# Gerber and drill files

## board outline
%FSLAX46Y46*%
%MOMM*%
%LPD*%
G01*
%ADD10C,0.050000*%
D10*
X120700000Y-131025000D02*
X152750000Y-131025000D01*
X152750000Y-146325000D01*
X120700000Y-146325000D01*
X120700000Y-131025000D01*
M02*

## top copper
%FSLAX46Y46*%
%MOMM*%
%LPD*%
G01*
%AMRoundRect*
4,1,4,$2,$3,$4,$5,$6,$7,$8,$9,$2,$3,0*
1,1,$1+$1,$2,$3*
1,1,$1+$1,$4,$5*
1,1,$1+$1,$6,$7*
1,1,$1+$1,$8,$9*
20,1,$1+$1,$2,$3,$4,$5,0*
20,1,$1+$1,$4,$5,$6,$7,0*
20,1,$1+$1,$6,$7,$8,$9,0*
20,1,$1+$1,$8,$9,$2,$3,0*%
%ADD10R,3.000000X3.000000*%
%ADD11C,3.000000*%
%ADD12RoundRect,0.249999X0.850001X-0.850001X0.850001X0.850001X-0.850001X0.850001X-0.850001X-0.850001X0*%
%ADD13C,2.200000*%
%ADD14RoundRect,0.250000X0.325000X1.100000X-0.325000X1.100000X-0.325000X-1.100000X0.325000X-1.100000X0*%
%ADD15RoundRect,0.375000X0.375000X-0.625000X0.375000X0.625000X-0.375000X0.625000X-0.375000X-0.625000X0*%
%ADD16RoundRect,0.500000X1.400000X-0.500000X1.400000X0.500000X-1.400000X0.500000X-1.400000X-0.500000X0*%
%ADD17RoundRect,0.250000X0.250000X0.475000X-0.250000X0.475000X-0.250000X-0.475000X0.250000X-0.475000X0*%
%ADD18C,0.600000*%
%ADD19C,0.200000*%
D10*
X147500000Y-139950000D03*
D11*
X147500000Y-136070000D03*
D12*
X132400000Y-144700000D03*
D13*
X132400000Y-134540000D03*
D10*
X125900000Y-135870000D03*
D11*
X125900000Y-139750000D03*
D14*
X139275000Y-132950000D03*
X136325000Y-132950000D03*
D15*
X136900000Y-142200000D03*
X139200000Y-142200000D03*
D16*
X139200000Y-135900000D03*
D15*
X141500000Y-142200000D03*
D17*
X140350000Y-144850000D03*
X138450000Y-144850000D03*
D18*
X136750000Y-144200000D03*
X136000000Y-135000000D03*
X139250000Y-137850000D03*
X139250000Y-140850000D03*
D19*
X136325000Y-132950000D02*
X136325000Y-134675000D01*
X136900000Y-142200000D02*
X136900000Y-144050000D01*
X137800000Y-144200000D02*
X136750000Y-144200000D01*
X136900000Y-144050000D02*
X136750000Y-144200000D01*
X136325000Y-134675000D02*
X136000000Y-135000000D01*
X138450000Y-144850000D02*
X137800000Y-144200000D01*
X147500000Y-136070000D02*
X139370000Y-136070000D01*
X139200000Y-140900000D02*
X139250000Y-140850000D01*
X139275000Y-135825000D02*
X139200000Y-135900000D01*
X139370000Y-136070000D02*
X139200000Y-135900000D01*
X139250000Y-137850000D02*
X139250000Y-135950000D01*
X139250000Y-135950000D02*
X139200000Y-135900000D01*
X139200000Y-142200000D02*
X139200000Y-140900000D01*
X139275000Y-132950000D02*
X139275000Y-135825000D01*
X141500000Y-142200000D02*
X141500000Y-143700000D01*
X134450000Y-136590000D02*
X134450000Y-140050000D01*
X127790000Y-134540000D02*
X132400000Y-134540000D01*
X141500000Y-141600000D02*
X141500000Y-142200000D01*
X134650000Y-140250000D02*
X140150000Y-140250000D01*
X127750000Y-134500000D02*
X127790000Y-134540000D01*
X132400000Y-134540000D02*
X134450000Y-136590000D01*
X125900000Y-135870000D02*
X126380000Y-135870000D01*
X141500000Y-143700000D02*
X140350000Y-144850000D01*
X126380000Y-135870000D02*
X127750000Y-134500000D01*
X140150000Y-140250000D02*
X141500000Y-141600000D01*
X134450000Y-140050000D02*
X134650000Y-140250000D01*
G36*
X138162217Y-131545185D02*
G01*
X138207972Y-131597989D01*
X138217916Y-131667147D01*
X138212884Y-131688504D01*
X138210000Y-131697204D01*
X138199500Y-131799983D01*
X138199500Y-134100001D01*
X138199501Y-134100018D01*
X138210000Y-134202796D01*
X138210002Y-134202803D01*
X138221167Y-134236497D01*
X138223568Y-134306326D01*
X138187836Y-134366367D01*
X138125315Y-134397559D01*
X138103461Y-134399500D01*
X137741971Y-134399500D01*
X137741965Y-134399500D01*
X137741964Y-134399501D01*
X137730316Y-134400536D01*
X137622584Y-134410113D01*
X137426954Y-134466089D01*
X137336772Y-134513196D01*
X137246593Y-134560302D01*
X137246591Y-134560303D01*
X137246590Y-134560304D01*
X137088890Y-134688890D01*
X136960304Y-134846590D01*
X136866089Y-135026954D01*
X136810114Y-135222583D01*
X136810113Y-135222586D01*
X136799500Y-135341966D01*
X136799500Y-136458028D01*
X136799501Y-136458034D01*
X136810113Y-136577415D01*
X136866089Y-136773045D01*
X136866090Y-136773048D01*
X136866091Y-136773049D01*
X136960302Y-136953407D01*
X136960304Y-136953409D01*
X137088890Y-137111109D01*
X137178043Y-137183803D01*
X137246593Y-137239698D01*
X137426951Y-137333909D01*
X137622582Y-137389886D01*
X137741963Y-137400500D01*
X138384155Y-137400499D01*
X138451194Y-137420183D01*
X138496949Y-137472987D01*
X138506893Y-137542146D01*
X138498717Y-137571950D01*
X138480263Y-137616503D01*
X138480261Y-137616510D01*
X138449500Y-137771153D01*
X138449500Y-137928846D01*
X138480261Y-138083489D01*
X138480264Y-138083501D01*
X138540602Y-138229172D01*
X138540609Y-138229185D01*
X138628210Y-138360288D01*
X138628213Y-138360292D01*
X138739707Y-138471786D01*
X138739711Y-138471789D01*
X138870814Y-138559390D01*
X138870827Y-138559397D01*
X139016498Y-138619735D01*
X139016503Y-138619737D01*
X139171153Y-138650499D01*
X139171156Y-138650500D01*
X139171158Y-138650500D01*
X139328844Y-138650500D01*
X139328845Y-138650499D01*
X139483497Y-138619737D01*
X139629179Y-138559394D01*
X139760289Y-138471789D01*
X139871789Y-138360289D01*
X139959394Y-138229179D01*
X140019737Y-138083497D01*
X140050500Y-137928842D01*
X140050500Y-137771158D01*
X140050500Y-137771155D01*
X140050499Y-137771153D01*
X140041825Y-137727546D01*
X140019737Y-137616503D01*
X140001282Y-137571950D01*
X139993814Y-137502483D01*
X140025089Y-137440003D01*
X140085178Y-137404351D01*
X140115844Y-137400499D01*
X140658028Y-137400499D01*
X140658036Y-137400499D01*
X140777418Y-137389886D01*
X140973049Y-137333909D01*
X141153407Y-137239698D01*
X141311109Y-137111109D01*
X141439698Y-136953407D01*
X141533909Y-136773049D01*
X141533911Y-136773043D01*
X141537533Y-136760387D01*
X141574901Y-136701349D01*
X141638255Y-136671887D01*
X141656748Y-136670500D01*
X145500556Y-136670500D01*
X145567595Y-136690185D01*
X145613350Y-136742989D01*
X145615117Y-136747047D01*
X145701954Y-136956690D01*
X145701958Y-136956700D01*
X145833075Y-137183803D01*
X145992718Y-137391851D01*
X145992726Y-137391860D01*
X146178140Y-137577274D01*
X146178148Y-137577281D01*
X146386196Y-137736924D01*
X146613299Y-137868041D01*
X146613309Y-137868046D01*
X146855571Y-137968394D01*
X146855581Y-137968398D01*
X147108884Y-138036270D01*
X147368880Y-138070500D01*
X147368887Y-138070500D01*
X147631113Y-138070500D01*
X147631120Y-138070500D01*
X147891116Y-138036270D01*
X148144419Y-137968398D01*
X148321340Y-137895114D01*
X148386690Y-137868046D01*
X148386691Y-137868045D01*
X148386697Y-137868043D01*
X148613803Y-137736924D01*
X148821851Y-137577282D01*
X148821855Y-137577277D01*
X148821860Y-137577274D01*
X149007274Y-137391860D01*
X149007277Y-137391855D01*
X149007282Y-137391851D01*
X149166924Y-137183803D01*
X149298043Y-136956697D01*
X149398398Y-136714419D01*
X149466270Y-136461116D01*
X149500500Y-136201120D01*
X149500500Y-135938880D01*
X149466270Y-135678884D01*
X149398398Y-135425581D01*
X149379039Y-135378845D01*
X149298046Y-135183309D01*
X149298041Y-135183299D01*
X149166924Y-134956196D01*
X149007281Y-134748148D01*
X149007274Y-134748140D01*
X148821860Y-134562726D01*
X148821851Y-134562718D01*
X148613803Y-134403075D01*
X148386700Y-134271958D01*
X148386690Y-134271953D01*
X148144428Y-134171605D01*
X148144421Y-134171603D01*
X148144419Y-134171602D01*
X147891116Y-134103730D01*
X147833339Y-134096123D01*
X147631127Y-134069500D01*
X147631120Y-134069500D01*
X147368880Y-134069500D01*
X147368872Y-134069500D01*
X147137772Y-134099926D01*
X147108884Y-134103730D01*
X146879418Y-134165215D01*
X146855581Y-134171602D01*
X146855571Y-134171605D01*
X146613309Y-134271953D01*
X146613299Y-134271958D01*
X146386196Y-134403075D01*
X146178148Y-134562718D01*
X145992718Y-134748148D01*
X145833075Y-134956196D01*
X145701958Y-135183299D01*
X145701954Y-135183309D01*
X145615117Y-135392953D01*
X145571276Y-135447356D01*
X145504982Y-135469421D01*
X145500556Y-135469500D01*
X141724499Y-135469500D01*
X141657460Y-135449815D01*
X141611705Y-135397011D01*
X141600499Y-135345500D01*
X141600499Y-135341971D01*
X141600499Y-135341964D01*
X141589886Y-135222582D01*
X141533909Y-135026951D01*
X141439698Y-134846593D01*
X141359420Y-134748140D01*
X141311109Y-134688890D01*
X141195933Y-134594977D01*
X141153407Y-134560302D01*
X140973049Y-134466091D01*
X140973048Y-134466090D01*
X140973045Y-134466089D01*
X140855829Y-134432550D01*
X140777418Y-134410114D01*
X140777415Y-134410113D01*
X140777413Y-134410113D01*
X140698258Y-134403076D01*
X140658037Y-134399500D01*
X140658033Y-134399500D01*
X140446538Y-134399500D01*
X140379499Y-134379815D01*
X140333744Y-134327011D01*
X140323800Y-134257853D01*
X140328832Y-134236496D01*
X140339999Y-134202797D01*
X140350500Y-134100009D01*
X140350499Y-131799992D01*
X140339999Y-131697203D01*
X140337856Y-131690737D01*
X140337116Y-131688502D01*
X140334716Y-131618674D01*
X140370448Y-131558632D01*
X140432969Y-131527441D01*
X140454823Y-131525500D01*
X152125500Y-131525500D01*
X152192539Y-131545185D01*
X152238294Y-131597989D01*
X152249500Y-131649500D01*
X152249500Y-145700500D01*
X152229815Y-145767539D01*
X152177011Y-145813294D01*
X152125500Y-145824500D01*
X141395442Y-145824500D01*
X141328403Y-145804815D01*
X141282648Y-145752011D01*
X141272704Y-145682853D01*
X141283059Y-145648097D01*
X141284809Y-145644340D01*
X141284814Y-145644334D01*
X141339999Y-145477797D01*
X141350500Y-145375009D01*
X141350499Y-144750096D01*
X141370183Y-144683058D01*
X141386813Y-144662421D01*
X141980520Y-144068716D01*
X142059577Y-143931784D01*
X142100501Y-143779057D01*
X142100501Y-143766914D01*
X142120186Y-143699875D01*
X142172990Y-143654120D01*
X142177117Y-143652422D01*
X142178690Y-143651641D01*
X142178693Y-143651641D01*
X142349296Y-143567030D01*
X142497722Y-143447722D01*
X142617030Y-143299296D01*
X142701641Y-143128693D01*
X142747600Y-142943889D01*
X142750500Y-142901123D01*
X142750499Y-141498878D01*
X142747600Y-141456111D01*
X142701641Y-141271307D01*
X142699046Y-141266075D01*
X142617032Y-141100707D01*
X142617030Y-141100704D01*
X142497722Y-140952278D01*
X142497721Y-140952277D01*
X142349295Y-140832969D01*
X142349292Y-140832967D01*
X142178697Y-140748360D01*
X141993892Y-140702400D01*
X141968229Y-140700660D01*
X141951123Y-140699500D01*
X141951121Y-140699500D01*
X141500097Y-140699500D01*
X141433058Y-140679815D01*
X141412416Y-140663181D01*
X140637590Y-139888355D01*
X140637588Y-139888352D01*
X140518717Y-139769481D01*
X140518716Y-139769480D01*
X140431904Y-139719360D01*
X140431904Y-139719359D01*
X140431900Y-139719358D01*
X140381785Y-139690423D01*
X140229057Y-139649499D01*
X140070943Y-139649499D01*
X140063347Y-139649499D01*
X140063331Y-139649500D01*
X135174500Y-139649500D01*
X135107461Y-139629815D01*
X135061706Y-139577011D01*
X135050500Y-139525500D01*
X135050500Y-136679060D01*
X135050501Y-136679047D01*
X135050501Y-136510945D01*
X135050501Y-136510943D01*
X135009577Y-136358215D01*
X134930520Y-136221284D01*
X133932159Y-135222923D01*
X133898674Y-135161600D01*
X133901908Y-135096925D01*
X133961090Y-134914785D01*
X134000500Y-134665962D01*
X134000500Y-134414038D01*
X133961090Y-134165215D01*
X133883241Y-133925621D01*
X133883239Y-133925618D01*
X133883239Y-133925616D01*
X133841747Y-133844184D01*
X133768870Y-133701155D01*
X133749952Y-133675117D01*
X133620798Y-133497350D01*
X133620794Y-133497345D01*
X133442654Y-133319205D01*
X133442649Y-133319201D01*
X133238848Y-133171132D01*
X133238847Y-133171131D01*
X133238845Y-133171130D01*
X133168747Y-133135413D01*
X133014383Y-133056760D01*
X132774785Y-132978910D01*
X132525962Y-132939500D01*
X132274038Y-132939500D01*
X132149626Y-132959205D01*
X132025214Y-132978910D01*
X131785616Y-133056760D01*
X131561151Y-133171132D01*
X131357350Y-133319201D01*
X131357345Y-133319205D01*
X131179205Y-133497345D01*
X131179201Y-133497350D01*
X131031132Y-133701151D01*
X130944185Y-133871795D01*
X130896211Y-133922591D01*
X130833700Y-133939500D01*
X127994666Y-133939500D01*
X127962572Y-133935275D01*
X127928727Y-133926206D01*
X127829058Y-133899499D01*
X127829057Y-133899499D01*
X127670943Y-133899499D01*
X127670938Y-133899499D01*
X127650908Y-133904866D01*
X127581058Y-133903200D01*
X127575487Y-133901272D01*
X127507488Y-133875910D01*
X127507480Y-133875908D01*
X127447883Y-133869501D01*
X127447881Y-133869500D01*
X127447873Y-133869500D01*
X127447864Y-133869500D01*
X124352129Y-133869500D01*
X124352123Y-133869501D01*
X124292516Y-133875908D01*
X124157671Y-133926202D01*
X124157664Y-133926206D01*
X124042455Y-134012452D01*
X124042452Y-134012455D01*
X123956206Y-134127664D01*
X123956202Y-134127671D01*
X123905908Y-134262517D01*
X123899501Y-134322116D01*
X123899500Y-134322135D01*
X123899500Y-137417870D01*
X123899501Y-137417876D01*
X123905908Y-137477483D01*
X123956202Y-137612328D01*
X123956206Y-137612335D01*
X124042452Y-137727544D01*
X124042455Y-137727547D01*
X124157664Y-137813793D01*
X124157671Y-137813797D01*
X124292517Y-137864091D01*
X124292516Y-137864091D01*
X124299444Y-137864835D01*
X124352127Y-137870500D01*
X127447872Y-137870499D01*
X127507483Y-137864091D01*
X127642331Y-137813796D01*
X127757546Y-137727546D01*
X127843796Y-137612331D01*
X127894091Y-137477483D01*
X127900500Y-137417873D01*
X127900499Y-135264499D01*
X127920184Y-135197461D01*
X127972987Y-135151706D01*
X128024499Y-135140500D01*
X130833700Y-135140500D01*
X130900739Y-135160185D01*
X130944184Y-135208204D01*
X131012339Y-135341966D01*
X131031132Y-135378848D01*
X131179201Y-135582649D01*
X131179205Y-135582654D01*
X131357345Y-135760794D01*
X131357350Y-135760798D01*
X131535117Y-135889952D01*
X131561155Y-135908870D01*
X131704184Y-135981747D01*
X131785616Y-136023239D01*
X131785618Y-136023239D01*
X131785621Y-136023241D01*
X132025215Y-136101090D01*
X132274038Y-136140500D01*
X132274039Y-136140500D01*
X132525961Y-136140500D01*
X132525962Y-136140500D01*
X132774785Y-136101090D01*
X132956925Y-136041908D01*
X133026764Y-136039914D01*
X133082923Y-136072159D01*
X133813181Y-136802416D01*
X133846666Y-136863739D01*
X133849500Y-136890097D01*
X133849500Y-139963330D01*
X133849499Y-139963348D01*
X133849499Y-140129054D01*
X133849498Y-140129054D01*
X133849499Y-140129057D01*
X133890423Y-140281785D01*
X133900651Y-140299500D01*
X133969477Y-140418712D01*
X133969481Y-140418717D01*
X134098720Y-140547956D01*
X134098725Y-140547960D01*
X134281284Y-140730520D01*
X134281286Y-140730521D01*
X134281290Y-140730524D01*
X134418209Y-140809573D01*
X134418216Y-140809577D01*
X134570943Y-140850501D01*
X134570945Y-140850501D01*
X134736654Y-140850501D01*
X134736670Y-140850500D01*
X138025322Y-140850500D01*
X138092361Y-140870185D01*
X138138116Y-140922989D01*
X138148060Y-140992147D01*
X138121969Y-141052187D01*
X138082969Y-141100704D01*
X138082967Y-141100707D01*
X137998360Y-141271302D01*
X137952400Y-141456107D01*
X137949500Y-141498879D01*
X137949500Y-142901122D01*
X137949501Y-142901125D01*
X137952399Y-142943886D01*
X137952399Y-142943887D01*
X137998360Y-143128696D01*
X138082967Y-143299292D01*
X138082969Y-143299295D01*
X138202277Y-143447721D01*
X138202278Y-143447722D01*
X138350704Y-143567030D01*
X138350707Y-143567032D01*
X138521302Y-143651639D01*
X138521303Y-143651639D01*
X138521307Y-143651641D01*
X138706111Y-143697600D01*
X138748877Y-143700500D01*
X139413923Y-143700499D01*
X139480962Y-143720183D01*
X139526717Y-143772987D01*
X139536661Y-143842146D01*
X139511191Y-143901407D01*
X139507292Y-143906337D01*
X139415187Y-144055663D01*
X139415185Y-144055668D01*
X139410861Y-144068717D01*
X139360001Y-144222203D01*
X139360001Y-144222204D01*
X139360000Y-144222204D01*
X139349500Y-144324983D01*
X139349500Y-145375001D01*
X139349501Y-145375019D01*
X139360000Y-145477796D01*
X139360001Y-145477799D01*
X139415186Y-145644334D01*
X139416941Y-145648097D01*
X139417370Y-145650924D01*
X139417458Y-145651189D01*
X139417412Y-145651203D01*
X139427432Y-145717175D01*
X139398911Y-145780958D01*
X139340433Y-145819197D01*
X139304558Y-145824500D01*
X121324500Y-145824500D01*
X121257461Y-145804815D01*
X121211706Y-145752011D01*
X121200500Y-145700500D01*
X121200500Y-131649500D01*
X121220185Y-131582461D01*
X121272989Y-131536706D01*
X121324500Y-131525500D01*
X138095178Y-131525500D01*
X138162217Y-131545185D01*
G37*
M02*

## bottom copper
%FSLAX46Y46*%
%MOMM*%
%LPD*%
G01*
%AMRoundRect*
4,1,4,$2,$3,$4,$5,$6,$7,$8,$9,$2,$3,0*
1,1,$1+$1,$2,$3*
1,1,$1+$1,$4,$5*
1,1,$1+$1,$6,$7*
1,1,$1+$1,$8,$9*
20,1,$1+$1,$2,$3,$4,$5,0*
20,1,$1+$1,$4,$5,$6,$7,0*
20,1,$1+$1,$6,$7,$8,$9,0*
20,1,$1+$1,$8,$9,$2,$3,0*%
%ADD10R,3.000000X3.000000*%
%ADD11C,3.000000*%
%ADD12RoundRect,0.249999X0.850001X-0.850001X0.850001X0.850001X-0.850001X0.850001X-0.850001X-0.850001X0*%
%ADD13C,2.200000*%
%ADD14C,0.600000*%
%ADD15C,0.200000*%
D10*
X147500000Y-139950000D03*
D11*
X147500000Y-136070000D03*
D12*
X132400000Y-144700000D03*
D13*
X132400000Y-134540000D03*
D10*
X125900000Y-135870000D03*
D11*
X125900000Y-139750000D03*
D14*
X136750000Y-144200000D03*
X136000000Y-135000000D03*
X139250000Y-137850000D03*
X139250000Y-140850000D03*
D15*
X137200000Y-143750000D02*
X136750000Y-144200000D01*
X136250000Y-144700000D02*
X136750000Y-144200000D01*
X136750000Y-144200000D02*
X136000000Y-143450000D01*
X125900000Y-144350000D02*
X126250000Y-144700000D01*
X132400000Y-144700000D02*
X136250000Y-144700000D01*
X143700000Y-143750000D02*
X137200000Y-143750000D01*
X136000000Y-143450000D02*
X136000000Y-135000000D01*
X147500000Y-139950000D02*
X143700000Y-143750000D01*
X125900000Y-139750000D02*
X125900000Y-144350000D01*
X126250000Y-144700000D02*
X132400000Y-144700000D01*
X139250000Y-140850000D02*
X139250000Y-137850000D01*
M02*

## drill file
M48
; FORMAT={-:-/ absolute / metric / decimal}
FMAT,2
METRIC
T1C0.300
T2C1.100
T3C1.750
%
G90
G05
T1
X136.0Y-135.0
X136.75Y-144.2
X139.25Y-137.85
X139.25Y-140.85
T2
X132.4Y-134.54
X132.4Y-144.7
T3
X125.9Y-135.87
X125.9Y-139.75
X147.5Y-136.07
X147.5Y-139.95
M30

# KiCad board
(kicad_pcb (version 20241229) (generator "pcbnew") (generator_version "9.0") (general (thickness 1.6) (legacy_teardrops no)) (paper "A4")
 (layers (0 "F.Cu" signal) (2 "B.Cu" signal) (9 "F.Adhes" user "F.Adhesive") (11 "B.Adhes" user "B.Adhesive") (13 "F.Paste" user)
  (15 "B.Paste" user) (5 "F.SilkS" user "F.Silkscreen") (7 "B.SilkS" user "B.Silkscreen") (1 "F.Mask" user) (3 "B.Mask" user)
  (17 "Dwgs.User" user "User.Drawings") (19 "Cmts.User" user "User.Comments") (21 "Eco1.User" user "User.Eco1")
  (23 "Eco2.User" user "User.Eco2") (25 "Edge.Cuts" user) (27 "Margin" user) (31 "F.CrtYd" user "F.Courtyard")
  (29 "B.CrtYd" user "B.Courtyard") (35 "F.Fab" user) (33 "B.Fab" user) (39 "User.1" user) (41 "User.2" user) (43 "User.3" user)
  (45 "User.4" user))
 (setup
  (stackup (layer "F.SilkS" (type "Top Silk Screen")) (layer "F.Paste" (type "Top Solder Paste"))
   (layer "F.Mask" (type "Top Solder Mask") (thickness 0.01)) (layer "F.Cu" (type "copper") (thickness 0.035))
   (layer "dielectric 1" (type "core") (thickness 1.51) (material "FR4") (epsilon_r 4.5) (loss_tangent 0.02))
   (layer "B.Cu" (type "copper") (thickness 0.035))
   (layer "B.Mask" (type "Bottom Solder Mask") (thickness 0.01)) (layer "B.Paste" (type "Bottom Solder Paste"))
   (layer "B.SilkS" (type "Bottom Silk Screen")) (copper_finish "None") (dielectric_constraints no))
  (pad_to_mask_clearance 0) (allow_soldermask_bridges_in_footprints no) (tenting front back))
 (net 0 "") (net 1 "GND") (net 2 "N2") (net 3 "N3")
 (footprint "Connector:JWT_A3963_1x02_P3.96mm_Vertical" (layer "F.Cu") (at 147.5 139.95 90)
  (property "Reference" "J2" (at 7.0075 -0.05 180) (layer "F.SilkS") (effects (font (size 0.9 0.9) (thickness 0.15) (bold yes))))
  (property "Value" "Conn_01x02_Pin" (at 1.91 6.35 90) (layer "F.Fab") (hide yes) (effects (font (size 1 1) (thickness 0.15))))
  (pad "1" thru_hole rect (at 0 0 90) (size 3 3) (drill 1.75) (layers "*.Cu" "*.Mask") (remove_unused_layers no) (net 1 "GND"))
  (pad "2" thru_hole circle (at 3.88 0 90) (size 3 3) (drill 1.75) (layers "*.Cu" "*.Mask") (remove_unused_layers no) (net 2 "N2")))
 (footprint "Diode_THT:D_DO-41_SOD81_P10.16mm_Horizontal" (layer "F.Cu") (at 132.4 144.7 90)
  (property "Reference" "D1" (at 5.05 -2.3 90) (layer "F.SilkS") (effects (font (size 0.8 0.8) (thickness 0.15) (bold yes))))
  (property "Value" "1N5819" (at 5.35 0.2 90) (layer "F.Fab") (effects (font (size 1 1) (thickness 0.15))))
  (pad "1" thru_hole roundrect (at 0 0 90) (size 2.2 2.2) (drill 1.1) (layers "*.Cu" "*.Mask") (remove_unused_layers no)
   (roundrect_rratio 0.113636) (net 1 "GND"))
  (pad "2" thru_hole circle (at 10.16 0 90) (size 2.2 2.2) (drill 1.1) (layers "*.Cu" "*.Mask") (remove_unused_layers no) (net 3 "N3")))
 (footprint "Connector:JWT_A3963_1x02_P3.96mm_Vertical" (layer "F.Cu") (at 125.9 135.87 -90)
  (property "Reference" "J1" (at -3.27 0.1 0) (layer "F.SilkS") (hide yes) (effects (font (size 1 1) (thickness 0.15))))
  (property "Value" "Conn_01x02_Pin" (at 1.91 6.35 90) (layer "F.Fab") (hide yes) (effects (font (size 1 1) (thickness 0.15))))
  (pad "1" thru_hole rect (at 0 0 270) (size 3 3) (drill 1.75) (layers "*.Cu" "*.Mask") (remove_unused_layers no) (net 3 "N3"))
  (pad "2" thru_hole circle (at 3.88 0 270) (size 3 3) (drill 1.75) (layers "*.Cu" "*.Mask") (remove_unused_layers no) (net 1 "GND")))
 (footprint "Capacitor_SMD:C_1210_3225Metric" (layer "F.Cu") (at 137.8 132.95 180)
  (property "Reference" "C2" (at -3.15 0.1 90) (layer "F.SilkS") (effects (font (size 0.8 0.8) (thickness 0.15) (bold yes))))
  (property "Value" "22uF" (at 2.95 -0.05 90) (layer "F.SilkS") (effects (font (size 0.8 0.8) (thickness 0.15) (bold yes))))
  (pad "1" smd roundrect (at -1.475 0 180) (size 1.15 2.7) (layers "F.Cu" "F.Mask" "F.Paste") (roundrect_rratio 0.217391) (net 2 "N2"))
  (pad "2" smd roundrect (at 1.475 0 180) (size 1.15 2.7) (layers "F.Cu" "F.Mask" "F.Paste") (roundrect_rratio 0.217391) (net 1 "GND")))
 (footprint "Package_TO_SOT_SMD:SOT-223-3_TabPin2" (layer "F.Cu") (at 139.2 139.05 90)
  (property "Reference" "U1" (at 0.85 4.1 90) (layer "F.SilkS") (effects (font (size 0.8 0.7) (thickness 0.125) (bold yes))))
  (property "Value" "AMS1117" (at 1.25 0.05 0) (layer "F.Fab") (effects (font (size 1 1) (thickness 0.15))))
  (pad "1" smd roundrect (at -3.15 -2.3 90) (size 2 1.5) (layers "F.Cu" "F.Mask" "F.Paste") (roundrect_rratio 0.25) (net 1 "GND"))
  (pad "2" smd roundrect (at -3.15 0 90) (size 2 1.5) (layers "F.Cu" "F.Mask" "F.Paste") (roundrect_rratio 0.25) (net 2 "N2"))
  (pad "2" smd roundrect (at 3.15 0 90) (size 2 3.8) (layers "F.Cu" "F.Mask" "F.Paste") (roundrect_rratio 0.25) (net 2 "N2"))
  (pad "3" smd roundrect (at -3.15 2.3 90) (size 2 1.5) (layers "F.Cu" "F.Mask" "F.Paste") (roundrect_rratio 0.25) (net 3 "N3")))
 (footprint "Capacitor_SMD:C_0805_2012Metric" (layer "F.Cu") (at 139.4 144.85 180)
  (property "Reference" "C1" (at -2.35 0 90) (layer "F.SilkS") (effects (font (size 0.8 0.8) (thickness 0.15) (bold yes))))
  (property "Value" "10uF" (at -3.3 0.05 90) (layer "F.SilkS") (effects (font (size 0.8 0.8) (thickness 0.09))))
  (pad "1" smd roundrect (at -0.95 0 180) (size 1 1.45) (layers "F.Cu" "F.Mask" "F.Paste") (roundrect_rratio 0.25) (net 3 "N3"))
  (pad "2" smd roundrect (at 0.95 0 180) (size 1 1.45) (layers "F.Cu" "F.Mask" "F.Paste") (roundrect_rratio 0.25) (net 1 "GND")))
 (gr_rect (start 120.7 131.025) (end 152.75 146.325) (stroke (width 0.05) (type default)) (fill no) (layer "Edge.Cuts"))
 (segment (start 136.325 132.95) (end 136.325 134.675) (width 0.2) (layer "F.Cu") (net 1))
 (segment (start 136.9 142.2) (end 136.9 144.05) (width 0.2) (layer "F.Cu") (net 1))
 (segment (start 137.8 144.2) (end 136.75 144.2) (width 0.2) (layer "F.Cu") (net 1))
 (segment (start 136.9 144.05) (end 136.75 144.2) (width 0.2) (layer "F.Cu") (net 1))
 (segment (start 136.325 134.675) (end 136 135) (width 0.2) (layer "F.Cu") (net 1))
 (segment (start 138.45 144.85) (end 137.8 144.2) (width 0.2) (layer "F.Cu") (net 1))
 (via (at 136.75 144.2) (size 0.6) (drill 0.3) (layers "F.Cu" "B.Cu") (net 1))
 (via (at 136 135) (size 0.6) (drill 0.3) (layers "F.Cu" "B.Cu") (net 1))
 (segment (start 137.2 143.75) (end 136.75 144.2) (width 0.2) (layer "B.Cu") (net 1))
 (segment (start 136.25 144.7) (end 136.75 144.2) (width 0.2) (layer "B.Cu") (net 1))
 (segment (start 136.75 144.2) (end 136 143.45) (width 0.2) (layer "B.Cu") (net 1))
 (segment (start 125.9 144.35) (end 126.25 144.7) (width 0.2) (layer "B.Cu") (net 1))
 (segment (start 132.4 144.7) (end 136.25 144.7) (width 0.2) (layer "B.Cu") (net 1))
 (segment (start 143.7 143.75) (end 137.2 143.75) (width 0.2) (layer "B.Cu") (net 1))
 (segment (start 136 143.45) (end 136 135) (width 0.2) (layer "B.Cu") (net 1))
 (segment (start 147.5 139.95) (end 143.7 143.75) (width 0.2) (layer "B.Cu") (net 1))
 (segment (start 125.9 139.75) (end 125.9 144.35) (width 0.2) (layer "B.Cu") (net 1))
 (segment (start 126.25 144.7) (end 132.4 144.7) (width 0.2) (layer "B.Cu") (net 1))
 (segment (start 147.5 136.07) (end 139.37 136.07) (width 0.2) (layer "F.Cu") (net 2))
 (segment (start 139.2 140.9) (end 139.25 140.85) (width 0.2) (layer "F.Cu") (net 2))
 (segment (start 139.275 135.825) (end 139.2 135.9) (width 0.2) (layer "F.Cu") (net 2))
 (segment (start 139.37 136.07) (end 139.2 135.9) (width 0.2) (layer "F.Cu") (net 2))
 (segment (start 139.25 137.85) (end 139.25 135.95) (width 0.2) (layer "F.Cu") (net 2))
 (segment (start 139.25 135.95) (end 139.2 135.9) (width 0.2) (layer "F.Cu") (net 2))
 (segment (start 139.2 142.2) (end 139.2 140.9) (width 0.2) (layer "F.Cu") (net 2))
 (segment (start 139.275 132.95) (end 139.275 135.825) (width 0.2) (layer "F.Cu") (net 2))
 (via (at 139.25 137.85) (size 0.6) (drill 0.3) (layers "F.Cu" "B.Cu") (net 2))
 (via (at 139.25 140.85) (size 0.6) (drill 0.3) (layers "F.Cu" "B.Cu") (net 2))
 (segment (start 139.25 140.85) (end 139.25 137.85) (width 0.2) (layer "B.Cu") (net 2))
 (segment (start 141.5 142.2) (end 141.5 143.7) (width 0.2) (layer "F.Cu") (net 3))
 (segment (start 134.45 136.59) (end 134.45 140.05) (width 0.2) (layer "F.Cu") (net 3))
 (segment (start 127.79 134.54) (end 132.4 134.54) (width 0.2) (layer "F.Cu") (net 3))
 (segment (start 141.5 141.6) (end 141.5 142.2) (width 0.2) (layer "F.Cu") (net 3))
 (segment (start 134.65 140.25) (end 140.15 140.25) (width 0.2) (layer "F.Cu") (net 3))
 (segment (start 127.75 134.5) (end 127.79 134.54) (width 0.2) (layer "F.Cu") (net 3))
 (segment (start 132.4 134.54) (end 134.45 136.59) (width 0.2) (layer "F.Cu") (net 3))
 (segment (start 125.9 135.87) (end 126.38 135.87) (width 0.2) (layer "F.Cu") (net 3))
 (segment (start 141.5 143.7) (end 140.35 144.85) (width 0.2) (layer "F.Cu") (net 3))
 (segment (start 126.38 135.87) (end 127.75 134.5) (width 0.2) (layer "F.Cu") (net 3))
 (segment (start 140.15 140.25) (end 141.5 141.6) (width 0.2) (layer "F.Cu") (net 3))
 (segment (start 134.45 140.05) (end 134.65 140.25) (width 0.2) (layer "F.Cu") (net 3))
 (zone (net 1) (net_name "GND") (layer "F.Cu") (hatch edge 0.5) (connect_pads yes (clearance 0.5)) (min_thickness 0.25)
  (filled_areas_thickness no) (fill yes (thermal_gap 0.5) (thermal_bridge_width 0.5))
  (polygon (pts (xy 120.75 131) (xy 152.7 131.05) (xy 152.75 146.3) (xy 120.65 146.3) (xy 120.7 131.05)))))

